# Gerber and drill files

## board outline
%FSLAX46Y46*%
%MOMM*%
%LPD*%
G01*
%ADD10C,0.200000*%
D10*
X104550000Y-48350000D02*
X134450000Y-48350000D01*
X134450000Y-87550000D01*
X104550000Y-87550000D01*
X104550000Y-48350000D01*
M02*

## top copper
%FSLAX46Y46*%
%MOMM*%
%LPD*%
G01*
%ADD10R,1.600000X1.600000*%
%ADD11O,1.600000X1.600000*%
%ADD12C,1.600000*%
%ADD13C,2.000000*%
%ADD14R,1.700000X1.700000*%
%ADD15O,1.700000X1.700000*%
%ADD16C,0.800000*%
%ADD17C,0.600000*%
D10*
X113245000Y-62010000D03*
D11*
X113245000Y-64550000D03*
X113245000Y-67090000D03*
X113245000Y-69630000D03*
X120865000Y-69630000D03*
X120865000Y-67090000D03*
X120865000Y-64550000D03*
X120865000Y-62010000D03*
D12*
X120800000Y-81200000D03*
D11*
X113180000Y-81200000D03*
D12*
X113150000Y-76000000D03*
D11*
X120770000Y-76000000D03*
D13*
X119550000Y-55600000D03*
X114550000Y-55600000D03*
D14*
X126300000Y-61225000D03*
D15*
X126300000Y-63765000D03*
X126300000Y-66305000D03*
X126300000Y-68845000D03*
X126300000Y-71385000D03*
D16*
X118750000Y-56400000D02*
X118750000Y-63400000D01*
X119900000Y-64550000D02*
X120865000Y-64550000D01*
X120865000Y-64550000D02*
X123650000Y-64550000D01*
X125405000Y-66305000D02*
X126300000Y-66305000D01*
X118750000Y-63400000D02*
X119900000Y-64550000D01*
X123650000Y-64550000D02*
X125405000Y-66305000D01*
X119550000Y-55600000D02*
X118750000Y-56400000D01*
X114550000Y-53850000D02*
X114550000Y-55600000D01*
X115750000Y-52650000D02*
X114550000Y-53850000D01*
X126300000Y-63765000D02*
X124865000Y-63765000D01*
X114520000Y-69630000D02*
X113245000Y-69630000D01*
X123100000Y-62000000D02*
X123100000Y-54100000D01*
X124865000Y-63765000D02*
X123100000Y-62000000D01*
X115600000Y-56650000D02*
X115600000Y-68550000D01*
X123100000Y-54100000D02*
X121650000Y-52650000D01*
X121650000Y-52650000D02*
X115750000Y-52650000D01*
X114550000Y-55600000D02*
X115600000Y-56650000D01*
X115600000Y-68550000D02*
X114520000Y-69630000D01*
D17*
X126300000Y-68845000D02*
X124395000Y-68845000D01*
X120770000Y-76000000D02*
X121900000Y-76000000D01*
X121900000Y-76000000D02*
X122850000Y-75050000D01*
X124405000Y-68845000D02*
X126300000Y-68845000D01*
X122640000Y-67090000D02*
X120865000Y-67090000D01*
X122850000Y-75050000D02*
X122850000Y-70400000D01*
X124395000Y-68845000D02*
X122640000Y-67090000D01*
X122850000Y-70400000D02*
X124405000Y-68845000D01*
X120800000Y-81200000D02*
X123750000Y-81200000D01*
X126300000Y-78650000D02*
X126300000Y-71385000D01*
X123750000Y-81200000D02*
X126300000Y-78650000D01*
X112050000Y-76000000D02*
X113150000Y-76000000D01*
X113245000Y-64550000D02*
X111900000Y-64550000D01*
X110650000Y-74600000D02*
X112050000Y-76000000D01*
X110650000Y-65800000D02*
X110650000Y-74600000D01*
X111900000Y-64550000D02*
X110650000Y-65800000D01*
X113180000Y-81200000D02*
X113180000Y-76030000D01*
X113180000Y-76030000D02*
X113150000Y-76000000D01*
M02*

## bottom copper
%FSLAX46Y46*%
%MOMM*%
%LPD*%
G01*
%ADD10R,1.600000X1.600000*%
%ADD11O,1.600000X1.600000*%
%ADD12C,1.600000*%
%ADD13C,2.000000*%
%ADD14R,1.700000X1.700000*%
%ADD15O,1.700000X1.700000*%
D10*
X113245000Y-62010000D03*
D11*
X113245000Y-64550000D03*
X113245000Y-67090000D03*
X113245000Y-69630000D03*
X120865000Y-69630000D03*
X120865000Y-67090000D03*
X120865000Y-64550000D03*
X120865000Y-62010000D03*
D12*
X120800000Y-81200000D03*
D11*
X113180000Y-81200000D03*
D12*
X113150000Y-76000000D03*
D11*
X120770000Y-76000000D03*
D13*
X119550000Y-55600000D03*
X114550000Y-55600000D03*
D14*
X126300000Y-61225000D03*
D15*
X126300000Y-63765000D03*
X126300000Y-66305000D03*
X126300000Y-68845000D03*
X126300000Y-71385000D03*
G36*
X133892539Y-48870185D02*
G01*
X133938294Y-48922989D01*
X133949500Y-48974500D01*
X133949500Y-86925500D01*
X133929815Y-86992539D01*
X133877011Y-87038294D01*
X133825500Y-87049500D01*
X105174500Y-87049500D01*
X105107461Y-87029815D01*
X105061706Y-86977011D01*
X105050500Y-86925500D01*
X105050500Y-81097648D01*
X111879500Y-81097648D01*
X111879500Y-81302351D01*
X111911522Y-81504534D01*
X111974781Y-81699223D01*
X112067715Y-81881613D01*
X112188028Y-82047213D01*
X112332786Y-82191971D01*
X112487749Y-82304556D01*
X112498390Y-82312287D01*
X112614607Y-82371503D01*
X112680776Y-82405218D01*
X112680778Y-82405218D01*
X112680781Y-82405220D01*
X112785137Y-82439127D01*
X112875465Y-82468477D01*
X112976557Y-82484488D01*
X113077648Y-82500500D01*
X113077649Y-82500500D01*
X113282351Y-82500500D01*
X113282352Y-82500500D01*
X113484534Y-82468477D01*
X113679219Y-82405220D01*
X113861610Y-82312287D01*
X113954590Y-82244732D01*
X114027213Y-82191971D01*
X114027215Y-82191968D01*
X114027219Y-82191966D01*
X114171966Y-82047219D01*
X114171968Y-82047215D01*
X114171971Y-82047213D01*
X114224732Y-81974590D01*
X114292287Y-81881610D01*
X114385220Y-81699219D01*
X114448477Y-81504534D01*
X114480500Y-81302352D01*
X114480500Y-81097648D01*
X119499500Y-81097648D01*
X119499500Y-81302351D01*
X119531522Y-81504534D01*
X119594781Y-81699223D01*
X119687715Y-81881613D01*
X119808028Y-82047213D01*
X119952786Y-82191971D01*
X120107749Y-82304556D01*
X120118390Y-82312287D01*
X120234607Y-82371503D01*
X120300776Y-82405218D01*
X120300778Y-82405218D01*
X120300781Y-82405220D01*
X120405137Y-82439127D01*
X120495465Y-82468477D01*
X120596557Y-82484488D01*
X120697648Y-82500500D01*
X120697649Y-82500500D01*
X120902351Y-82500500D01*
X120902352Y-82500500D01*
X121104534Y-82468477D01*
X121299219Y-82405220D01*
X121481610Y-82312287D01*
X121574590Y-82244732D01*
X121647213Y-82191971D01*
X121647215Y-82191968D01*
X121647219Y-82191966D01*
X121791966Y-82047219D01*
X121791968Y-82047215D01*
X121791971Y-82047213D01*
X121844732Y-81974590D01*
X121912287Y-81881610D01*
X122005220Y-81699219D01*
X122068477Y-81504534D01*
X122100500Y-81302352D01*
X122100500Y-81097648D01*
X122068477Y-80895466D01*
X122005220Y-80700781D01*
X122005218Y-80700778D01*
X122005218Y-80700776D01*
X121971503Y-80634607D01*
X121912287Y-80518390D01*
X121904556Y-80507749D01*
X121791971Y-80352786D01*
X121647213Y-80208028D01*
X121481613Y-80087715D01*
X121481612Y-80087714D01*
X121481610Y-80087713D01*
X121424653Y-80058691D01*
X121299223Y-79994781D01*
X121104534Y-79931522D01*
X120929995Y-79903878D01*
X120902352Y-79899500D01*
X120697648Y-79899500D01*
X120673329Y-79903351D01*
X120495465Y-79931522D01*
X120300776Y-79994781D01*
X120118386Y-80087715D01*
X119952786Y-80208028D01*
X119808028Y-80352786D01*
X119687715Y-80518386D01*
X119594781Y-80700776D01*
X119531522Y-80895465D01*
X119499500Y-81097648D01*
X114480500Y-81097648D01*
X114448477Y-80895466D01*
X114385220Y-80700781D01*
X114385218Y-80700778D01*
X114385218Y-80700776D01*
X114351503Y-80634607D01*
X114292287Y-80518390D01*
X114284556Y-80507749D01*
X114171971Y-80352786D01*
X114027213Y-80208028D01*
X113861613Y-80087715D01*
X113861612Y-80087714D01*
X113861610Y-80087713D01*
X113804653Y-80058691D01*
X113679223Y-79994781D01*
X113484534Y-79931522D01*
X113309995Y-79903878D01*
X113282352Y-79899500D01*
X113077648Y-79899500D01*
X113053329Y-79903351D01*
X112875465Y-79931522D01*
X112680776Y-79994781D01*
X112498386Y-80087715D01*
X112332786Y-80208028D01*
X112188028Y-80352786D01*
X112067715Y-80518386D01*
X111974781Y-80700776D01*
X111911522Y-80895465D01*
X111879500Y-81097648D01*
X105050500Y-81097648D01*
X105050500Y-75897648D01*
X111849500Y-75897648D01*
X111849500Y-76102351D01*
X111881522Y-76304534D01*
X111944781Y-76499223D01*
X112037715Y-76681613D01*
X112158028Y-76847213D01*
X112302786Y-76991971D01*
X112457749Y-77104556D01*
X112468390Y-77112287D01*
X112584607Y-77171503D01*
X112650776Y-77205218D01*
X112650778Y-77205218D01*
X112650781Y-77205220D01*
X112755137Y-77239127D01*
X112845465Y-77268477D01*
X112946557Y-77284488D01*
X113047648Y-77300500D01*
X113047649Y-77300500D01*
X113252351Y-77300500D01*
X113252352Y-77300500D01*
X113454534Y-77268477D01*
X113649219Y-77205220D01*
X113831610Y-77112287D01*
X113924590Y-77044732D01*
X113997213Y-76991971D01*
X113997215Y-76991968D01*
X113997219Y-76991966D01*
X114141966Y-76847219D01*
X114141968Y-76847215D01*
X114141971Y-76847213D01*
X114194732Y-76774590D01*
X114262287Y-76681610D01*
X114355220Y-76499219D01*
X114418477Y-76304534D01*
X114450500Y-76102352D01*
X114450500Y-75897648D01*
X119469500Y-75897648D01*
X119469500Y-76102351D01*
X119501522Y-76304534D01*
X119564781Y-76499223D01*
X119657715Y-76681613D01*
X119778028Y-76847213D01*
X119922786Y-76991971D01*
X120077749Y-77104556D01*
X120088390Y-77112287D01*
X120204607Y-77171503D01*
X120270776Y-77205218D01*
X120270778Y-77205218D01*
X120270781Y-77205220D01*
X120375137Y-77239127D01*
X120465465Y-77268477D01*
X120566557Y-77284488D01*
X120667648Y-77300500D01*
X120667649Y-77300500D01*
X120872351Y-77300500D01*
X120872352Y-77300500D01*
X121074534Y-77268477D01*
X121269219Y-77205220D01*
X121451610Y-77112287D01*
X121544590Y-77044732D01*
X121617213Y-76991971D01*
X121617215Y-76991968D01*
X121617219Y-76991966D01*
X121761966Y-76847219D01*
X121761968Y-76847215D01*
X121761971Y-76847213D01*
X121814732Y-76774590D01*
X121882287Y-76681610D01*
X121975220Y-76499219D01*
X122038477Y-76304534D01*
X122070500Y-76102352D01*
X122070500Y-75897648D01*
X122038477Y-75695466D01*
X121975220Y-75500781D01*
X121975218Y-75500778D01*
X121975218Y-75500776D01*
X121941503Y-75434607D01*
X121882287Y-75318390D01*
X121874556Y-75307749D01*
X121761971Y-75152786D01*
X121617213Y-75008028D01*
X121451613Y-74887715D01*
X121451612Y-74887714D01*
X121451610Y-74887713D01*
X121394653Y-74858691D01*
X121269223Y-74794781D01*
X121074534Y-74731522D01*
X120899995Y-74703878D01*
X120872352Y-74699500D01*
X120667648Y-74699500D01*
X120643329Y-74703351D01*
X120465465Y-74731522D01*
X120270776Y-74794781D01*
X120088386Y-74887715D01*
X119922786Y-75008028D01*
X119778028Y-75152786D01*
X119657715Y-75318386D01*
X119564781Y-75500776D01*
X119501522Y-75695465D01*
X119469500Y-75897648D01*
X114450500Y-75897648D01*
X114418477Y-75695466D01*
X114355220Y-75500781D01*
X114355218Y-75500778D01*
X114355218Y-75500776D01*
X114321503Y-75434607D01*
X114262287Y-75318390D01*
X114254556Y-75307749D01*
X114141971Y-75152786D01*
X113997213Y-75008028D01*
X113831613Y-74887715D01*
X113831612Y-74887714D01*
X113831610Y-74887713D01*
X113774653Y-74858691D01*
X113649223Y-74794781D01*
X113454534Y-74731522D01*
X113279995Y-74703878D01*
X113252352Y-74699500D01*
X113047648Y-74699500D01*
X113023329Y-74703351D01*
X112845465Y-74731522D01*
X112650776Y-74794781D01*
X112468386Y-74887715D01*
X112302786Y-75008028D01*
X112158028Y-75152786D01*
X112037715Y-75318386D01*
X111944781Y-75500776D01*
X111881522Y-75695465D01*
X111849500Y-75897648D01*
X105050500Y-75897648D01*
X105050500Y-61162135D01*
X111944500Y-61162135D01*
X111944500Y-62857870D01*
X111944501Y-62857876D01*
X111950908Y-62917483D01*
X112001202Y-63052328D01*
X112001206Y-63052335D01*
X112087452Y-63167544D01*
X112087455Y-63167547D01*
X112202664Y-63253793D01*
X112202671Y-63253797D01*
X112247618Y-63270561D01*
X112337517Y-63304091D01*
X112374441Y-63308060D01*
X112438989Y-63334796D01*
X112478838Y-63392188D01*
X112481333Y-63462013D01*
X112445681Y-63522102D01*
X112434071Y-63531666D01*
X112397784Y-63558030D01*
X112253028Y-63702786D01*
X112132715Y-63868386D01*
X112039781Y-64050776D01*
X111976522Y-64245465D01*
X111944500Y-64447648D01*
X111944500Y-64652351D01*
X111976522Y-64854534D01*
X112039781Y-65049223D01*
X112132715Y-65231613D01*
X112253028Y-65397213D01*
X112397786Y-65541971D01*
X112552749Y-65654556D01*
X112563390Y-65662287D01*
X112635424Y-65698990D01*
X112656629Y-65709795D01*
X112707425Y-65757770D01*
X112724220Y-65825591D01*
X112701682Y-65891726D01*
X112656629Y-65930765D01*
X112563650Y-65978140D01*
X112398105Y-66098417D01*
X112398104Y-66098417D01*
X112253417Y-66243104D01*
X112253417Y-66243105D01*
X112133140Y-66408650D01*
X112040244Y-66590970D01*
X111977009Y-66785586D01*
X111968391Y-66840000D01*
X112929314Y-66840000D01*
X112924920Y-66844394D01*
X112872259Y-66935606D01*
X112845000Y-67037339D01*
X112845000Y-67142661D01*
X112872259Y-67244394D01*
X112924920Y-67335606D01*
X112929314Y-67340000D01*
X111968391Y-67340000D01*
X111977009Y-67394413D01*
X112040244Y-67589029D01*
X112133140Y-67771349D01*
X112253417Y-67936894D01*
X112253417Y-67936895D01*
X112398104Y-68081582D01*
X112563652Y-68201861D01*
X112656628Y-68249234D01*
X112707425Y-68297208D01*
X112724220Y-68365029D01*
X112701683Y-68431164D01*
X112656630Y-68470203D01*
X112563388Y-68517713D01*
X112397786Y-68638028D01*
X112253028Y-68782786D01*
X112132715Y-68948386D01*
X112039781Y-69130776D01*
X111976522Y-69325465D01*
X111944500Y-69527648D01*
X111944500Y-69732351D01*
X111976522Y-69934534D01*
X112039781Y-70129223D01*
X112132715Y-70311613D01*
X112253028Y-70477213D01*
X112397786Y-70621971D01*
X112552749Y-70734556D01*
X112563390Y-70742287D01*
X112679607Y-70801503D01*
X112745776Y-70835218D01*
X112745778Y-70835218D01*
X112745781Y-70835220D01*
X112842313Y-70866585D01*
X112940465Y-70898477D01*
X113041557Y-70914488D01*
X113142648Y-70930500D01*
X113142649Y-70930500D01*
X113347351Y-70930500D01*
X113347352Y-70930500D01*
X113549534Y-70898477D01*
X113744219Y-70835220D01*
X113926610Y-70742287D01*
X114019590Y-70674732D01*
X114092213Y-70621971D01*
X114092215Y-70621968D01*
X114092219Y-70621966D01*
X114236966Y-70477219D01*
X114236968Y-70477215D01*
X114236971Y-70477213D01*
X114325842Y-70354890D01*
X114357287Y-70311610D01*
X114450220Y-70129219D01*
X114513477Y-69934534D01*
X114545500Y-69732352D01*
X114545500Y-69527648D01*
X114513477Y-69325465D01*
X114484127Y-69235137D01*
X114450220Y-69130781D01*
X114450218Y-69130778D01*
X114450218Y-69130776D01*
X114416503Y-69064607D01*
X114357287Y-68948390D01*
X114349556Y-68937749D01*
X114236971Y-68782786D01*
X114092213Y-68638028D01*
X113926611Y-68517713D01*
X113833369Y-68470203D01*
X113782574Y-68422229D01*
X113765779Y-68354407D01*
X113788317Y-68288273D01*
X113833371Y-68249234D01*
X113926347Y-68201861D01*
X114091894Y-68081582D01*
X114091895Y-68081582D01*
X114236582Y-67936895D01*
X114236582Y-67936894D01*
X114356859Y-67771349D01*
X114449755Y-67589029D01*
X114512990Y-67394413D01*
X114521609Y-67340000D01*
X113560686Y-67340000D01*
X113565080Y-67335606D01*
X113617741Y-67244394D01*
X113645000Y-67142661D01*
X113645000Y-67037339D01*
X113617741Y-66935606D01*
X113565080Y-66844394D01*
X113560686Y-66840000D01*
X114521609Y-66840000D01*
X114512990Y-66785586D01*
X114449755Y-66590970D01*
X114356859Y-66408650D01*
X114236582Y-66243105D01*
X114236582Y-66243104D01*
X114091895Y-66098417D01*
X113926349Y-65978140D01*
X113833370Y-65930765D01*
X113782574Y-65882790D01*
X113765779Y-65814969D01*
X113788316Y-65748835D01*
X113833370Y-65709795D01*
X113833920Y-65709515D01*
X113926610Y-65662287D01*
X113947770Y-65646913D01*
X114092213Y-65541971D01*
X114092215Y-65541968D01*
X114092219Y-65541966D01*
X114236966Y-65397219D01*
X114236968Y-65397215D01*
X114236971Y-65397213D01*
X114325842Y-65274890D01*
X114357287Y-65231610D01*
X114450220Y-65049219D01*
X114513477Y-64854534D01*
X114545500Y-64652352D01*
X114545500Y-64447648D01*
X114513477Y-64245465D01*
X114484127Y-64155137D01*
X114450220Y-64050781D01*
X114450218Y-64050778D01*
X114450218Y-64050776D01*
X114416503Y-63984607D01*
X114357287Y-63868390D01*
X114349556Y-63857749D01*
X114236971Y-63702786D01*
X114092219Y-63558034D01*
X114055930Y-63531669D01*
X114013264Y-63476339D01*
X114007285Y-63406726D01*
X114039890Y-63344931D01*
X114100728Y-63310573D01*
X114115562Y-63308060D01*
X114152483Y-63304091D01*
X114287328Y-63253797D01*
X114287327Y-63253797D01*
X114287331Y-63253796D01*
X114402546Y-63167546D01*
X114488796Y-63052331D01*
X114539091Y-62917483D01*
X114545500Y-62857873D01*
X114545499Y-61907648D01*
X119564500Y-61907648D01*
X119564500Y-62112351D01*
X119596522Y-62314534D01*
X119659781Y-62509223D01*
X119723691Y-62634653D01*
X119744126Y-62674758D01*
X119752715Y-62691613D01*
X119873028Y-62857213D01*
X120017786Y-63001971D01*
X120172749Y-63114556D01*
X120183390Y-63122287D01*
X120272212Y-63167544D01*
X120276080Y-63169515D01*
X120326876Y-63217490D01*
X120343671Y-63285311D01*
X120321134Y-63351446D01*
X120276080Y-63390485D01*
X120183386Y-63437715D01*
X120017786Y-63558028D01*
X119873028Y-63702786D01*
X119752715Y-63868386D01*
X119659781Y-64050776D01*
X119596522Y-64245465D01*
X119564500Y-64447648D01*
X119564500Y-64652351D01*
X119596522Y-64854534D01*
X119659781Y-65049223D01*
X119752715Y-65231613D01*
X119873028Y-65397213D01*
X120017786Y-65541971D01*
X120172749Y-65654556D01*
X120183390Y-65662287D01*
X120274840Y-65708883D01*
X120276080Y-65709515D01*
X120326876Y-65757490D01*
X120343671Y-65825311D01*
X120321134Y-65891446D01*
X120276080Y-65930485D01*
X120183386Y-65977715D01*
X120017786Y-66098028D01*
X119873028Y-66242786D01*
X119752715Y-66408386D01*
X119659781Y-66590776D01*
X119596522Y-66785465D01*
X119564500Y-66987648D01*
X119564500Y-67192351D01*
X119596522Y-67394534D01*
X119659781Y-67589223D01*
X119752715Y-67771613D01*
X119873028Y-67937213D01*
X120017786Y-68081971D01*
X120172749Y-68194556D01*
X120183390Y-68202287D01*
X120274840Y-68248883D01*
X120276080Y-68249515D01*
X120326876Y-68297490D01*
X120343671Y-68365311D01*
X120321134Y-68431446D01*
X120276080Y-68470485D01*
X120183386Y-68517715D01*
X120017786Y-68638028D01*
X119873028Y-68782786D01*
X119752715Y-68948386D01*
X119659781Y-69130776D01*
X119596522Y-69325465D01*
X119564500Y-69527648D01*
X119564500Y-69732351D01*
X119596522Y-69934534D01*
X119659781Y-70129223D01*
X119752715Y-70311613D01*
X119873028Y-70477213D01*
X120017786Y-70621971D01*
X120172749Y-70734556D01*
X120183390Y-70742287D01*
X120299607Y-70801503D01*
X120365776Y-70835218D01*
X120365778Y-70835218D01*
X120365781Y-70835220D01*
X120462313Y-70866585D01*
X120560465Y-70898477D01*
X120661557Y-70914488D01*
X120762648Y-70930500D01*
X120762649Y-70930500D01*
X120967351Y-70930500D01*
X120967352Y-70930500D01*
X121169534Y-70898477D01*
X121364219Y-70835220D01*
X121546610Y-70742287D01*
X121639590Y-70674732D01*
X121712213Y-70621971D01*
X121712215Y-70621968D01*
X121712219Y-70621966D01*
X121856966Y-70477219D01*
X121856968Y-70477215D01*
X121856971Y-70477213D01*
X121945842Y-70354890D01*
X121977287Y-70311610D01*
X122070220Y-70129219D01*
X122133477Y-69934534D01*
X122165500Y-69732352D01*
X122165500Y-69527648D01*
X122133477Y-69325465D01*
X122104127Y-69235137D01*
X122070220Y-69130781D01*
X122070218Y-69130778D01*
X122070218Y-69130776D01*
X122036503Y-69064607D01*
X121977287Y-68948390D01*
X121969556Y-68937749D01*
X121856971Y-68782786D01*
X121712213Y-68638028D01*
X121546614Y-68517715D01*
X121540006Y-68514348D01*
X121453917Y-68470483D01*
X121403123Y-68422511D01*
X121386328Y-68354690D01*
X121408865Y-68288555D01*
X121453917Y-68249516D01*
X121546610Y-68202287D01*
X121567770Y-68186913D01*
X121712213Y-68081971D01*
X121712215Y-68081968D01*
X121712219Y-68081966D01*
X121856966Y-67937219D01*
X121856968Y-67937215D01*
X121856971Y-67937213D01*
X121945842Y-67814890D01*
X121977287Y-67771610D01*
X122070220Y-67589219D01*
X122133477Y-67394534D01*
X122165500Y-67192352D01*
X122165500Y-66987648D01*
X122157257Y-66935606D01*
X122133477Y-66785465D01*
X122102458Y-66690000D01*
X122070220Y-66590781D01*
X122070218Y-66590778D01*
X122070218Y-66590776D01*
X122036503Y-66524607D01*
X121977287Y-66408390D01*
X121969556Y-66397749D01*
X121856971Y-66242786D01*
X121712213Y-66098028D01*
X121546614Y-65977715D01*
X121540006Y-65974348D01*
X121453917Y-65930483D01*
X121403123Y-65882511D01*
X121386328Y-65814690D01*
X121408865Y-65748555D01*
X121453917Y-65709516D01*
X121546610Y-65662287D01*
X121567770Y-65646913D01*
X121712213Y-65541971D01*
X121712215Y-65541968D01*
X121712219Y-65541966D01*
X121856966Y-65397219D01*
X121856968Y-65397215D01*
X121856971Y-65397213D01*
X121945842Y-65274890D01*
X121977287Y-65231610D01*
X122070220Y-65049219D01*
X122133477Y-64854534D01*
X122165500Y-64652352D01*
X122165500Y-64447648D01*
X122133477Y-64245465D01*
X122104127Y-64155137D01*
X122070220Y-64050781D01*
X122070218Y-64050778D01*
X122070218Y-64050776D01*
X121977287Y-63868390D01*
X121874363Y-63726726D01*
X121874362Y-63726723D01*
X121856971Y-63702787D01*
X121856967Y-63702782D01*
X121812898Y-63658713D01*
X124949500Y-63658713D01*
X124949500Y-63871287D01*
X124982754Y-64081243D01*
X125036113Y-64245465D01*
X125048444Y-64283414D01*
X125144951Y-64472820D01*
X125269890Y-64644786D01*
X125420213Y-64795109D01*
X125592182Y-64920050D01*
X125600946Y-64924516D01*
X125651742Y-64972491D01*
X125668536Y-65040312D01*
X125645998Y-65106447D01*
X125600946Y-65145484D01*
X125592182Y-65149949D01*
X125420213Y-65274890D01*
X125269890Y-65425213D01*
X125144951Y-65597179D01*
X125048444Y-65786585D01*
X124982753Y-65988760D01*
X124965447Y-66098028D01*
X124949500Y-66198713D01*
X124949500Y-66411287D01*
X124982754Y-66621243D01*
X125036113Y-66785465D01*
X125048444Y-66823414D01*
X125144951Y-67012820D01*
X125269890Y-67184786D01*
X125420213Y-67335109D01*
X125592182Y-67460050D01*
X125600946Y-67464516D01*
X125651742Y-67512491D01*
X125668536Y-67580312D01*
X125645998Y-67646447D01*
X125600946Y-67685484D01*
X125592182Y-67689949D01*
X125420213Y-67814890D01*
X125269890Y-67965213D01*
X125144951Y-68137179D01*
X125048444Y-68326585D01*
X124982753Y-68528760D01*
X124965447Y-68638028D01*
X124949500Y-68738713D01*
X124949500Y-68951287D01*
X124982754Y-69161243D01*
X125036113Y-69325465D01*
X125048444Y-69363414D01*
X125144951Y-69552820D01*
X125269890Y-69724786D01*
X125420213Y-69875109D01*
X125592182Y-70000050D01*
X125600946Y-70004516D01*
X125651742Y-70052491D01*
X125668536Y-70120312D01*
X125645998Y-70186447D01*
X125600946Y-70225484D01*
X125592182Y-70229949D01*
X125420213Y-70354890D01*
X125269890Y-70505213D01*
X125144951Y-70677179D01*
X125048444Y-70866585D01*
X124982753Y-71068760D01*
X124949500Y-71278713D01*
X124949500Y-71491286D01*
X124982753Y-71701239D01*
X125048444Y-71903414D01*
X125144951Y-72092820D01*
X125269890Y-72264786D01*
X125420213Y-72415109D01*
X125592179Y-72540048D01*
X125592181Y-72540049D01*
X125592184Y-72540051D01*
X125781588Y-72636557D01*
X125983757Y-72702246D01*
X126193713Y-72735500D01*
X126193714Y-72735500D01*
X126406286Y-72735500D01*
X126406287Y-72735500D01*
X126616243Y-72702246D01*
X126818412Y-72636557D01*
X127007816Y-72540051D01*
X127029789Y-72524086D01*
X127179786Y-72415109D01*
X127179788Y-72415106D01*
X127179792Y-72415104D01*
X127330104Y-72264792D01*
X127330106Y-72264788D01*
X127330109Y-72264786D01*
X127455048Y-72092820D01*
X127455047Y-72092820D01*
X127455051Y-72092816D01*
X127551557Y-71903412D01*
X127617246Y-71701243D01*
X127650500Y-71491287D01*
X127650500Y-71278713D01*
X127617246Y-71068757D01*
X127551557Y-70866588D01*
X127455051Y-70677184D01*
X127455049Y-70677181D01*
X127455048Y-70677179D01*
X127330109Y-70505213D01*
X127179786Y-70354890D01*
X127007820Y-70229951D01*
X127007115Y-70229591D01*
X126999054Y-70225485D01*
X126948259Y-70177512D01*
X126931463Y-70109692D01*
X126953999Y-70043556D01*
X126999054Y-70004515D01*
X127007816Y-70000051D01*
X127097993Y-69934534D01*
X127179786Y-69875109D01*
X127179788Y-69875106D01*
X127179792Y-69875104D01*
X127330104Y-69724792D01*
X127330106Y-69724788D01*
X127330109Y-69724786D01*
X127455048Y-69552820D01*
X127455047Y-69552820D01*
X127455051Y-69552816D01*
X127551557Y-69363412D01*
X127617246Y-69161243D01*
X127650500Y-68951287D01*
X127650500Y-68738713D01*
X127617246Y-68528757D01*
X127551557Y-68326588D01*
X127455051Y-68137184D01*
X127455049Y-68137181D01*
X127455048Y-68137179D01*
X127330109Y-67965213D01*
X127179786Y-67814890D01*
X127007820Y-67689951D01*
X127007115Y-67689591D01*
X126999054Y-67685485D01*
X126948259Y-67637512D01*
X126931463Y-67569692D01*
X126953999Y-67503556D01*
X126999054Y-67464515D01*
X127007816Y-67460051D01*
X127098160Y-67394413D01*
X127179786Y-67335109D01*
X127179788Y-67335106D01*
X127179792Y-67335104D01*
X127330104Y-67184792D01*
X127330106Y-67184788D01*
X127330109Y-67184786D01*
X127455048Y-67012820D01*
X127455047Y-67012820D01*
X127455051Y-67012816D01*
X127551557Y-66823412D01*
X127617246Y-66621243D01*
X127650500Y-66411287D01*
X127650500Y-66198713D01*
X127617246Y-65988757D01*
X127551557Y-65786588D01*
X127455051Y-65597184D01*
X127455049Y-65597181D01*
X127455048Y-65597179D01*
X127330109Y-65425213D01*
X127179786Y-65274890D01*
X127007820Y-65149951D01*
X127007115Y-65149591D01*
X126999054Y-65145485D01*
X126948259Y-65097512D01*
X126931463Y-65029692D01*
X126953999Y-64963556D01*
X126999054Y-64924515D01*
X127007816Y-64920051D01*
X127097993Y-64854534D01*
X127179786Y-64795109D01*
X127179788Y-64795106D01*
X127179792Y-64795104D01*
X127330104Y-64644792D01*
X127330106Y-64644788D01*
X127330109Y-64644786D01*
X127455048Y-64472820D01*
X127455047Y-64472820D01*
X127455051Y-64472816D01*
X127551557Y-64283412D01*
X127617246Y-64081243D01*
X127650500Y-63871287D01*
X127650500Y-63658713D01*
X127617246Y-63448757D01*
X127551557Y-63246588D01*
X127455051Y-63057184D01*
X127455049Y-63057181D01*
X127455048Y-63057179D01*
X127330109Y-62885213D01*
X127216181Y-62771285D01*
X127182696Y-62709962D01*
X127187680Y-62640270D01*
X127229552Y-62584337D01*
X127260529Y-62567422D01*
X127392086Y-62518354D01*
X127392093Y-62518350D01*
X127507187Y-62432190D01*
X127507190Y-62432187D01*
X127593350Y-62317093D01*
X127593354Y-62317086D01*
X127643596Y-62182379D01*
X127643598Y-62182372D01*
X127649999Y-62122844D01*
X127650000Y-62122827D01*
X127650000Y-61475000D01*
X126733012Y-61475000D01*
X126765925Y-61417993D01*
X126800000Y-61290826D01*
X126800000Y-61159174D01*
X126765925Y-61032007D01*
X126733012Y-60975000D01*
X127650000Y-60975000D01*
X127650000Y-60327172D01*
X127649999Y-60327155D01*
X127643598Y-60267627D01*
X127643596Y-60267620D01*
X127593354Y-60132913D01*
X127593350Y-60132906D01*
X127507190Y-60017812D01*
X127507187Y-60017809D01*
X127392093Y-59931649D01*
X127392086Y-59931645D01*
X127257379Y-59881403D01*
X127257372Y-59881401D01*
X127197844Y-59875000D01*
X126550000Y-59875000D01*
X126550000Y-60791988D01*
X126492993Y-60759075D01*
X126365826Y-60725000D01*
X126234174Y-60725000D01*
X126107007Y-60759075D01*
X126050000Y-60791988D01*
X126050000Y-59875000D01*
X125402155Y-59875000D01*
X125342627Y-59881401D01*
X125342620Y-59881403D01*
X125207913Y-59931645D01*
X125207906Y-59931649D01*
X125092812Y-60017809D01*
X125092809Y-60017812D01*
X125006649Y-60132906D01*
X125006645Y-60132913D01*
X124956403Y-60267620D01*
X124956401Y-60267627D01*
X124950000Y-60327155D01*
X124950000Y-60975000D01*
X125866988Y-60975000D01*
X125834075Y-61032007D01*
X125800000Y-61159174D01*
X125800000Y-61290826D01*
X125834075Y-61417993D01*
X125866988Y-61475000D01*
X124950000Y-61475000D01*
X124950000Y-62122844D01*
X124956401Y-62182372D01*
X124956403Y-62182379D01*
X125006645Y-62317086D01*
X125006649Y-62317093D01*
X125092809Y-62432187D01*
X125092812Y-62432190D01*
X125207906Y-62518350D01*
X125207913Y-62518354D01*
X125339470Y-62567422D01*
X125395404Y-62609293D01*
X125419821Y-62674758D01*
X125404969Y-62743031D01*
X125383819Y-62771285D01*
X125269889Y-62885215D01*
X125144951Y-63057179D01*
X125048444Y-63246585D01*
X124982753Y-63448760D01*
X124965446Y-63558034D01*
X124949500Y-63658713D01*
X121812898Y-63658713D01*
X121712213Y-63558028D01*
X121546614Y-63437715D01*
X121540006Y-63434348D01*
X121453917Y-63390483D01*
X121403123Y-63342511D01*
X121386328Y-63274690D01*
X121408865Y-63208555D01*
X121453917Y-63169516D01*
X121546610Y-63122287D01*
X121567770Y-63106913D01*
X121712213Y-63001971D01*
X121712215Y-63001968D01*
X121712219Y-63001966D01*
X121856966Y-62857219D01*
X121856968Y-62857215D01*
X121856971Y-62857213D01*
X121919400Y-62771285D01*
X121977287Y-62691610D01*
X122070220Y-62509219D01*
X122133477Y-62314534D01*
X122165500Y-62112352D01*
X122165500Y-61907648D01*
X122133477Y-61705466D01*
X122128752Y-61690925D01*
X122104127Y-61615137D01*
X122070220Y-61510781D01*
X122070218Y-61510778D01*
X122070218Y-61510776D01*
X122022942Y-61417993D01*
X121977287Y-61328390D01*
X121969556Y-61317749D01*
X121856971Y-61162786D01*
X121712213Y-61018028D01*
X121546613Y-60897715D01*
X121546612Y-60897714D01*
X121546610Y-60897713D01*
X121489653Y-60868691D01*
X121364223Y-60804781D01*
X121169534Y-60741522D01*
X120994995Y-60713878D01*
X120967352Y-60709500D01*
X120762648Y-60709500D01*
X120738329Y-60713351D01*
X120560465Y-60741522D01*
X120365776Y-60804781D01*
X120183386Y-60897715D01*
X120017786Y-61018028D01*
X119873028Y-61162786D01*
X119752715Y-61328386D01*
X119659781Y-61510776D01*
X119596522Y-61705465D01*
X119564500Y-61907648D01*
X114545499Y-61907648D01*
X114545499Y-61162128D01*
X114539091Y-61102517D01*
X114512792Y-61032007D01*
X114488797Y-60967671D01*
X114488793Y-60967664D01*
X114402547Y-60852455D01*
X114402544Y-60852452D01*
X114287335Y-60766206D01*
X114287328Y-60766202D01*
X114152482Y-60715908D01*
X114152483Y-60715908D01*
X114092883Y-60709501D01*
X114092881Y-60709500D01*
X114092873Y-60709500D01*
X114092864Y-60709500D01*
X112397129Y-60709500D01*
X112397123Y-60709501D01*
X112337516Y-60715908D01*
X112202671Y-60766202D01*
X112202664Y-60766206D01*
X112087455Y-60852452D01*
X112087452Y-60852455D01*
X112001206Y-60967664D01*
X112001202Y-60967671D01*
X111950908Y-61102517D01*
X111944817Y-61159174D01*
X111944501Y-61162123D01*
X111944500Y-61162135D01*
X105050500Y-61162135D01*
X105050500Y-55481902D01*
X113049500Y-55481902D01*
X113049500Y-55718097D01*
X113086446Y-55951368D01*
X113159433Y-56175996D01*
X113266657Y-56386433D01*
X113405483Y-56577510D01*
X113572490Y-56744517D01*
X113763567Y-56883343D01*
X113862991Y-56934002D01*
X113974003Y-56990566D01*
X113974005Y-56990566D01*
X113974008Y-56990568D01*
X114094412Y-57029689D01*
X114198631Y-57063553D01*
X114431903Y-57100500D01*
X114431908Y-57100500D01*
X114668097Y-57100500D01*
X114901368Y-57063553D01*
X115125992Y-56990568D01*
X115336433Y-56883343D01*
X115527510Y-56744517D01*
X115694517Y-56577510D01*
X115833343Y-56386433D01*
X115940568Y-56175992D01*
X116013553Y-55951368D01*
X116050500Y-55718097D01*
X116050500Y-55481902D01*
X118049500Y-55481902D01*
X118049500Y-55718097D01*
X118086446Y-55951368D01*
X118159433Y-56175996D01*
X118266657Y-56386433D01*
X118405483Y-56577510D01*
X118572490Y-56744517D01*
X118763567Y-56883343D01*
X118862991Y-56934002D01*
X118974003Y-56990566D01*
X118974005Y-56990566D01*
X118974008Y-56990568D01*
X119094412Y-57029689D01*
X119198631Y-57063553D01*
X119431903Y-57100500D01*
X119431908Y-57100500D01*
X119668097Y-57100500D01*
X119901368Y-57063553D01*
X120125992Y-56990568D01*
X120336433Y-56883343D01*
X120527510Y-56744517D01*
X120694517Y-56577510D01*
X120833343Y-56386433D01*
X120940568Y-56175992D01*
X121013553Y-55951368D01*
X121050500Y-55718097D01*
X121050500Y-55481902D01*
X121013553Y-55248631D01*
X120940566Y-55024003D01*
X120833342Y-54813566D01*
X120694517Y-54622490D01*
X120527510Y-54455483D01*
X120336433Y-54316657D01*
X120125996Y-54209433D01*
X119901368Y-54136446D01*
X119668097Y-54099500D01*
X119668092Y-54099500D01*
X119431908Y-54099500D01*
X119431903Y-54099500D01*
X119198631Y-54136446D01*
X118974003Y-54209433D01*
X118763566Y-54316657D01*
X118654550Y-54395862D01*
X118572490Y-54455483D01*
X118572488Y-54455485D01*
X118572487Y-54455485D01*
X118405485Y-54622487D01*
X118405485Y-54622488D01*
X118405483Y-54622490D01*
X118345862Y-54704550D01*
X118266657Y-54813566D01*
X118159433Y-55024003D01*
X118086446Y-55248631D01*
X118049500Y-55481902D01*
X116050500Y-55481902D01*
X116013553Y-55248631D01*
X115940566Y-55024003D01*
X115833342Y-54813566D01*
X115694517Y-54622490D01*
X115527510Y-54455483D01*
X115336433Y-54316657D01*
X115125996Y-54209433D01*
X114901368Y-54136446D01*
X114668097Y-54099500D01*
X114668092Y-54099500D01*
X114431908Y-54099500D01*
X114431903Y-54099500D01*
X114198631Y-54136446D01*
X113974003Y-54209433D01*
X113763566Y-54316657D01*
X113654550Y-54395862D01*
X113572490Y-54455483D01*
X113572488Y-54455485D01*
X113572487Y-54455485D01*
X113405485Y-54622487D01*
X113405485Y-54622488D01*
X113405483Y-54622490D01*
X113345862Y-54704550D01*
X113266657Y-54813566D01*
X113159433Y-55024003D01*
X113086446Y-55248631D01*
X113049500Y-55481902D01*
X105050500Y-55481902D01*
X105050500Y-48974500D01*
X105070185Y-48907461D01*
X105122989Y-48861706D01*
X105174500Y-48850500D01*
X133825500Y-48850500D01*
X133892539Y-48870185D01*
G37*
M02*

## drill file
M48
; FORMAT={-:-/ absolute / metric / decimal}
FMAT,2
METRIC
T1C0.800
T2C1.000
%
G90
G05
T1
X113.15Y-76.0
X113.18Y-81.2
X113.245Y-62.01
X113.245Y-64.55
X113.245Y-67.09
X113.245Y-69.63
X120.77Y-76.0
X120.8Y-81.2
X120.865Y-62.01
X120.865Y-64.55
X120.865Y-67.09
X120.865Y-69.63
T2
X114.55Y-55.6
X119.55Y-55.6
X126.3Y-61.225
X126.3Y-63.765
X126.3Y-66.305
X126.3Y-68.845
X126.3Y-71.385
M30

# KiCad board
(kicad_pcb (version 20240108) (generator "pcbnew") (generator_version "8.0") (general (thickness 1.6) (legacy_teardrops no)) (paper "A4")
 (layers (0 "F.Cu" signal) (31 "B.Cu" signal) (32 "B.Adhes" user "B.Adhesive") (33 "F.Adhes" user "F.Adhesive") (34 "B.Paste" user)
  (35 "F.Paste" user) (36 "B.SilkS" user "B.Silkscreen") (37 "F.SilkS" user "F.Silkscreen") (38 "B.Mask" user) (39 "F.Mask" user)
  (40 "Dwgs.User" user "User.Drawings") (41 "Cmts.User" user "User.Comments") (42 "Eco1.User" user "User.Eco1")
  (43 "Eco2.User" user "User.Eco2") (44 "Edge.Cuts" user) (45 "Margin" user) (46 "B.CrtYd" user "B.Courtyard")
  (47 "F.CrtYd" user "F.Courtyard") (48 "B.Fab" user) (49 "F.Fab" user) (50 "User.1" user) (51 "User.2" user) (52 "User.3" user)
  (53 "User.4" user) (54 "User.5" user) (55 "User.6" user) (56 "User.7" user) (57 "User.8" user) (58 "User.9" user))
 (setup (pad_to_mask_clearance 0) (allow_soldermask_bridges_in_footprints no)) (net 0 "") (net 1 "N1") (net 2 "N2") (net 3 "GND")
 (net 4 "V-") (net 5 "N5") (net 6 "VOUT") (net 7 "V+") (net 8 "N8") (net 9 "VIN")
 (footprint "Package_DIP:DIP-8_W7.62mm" (layer "F.Cu") (at 113.245 62.01)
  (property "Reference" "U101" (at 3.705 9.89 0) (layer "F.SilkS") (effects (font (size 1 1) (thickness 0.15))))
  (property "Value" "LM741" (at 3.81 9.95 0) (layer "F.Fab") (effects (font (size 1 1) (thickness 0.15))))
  (pad "1" thru_hole rect (at 0 0) (size 1.6 1.6) (drill 0.8) (layers "*.Cu" "*.Mask") (remove_unused_layers no) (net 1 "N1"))
  (pad "2" thru_hole oval (at 0 2.54) (size 1.6 1.6) (drill 0.8) (layers "*.Cu" "*.Mask") (remove_unused_layers no) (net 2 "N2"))
  (pad "3" thru_hole oval (at 0 5.08) (size 1.6 1.6) (drill 0.8) (layers "*.Cu" "*.Mask") (remove_unused_layers no) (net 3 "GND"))
  (pad "4" thru_hole oval (at 0 7.62) (size 1.6 1.6) (drill 0.8) (layers "*.Cu" "*.Mask") (remove_unused_layers no) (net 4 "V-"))
  (pad "5" thru_hole oval (at 7.62 7.62) (size 1.6 1.6) (drill 0.8) (layers "*.Cu" "*.Mask") (remove_unused_layers no) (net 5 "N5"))
  (pad "6" thru_hole oval (at 7.62 5.08) (size 1.6 1.6) (drill 0.8) (layers "*.Cu" "*.Mask") (remove_unused_layers no) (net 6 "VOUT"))
  (pad "7" thru_hole oval (at 7.62 2.54) (size 1.6 1.6) (drill 0.8) (layers "*.Cu" "*.Mask") (remove_unused_layers no) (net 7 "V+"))
  (pad "8" thru_hole oval (at 7.62 0) (size 1.6 1.6) (drill 0.8) (layers "*.Cu" "*.Mask") (remove_unused_layers no) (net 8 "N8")))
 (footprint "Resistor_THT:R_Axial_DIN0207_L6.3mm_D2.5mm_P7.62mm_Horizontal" (layer "F.Cu") (at 120.8 81.2 180)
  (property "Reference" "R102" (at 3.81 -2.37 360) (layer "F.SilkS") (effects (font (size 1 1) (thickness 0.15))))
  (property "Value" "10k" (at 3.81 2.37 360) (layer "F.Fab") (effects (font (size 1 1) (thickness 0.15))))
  (pad "1" thru_hole circle (at 0 0 180) (size 1.6 1.6) (drill 0.8) (layers "*.Cu" "*.Mask") (remove_unused_layers no) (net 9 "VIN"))
  (pad "2" thru_hole oval (at 7.62 0 180) (size 1.6 1.6) (drill 0.8) (layers "*.Cu" "*.Mask") (remove_unused_layers no) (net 2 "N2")))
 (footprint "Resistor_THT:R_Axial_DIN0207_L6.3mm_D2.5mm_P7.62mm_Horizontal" (layer "F.Cu") (at 113.15 76)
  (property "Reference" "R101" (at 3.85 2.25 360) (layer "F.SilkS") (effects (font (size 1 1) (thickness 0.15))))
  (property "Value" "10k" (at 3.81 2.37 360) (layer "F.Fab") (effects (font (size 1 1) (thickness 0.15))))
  (pad "1" thru_hole circle (at 0 0) (size 1.6 1.6) (drill 0.8) (layers "*.Cu" "*.Mask") (remove_unused_layers no) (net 2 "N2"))
  (pad "2" thru_hole oval (at 7.62 0) (size 1.6 1.6) (drill 0.8) (layers "*.Cu" "*.Mask") (remove_unused_layers no) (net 6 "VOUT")))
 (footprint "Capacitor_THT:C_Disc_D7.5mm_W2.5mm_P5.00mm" (layer "F.Cu") (at 119.55 55.6 180)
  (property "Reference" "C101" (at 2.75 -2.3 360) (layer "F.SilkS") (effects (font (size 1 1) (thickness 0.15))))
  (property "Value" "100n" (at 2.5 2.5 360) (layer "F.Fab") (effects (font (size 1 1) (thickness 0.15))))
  (pad "1" thru_hole circle (at 0 0 180) (size 2 2) (drill 1) (layers "*.Cu" "*.Mask") (remove_unused_layers no) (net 7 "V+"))
  (pad "2" thru_hole circle (at 5 0 180) (size 2 2) (drill 1) (layers "*.Cu" "*.Mask") (remove_unused_layers no) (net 4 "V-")))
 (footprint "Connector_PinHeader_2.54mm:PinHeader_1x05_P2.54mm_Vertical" (layer "F.Cu") (at 126.3 61.225)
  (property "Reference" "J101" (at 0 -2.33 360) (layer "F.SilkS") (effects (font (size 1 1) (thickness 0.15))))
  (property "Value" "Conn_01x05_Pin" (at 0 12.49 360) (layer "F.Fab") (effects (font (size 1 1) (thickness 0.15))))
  (pad "1" thru_hole rect (at 0 0) (size 1.7 1.7) (drill 1) (layers "*.Cu" "*.Mask") (remove_unused_layers no) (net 3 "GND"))
  (pad "2" thru_hole oval (at 0 2.54) (size 1.7 1.7) (drill 1) (layers "*.Cu" "*.Mask") (remove_unused_layers no) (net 4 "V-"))
  (pad "3" thru_hole oval (at 0 5.08) (size 1.7 1.7) (drill 1) (layers "*.Cu" "*.Mask") (remove_unused_layers no) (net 7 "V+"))
  (pad "4" thru_hole oval (at 0 7.62) (size 1.7 1.7) (drill 1) (layers "*.Cu" "*.Mask") (remove_unused_layers no) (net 6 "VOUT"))
  (pad "5" thru_hole oval (at 0 10.16) (size 1.7 1.7) (drill 1) (layers "*.Cu" "*.Mask") (remove_unused_layers no) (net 9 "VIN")))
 (gr_rect (start 104.55 48.35) (end 134.45 87.55) (stroke (width 0.2) (type default)) (fill none) (layer "Edge.Cuts"))
 (segment (start 118.75 56.4) (end 118.75 63.4) (width 0.8) (layer "F.Cu") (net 7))
 (segment (start 119.9 64.55) (end 120.865 64.55) (width 0.8) (layer "F.Cu") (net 7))
 (segment (start 120.865 64.55) (end 123.65 64.55) (width 0.8) (layer "F.Cu") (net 7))
 (segment (start 125.405 66.305) (end 126.3 66.305) (width 0.8) (layer "F.Cu") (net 7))
 (segment (start 118.75 63.4) (end 119.9 64.55) (width 0.8) (layer "F.Cu") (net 7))
 (segment (start 123.65 64.55) (end 125.405 66.305) (width 0.8) (layer "F.Cu") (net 7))
 (segment (start 119.55 55.6) (end 118.75 56.4) (width 0.8) (layer "F.Cu") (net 7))
 (segment (start 114.55 53.85) (end 114.55 55.6) (width 0.8) (layer "F.Cu") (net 4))
 (segment (start 115.75 52.65) (end 114.55 53.85) (width 0.8) (layer "F.Cu") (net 4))
 (segment (start 126.3 63.765) (end 124.865 63.765) (width 0.8) (layer "F.Cu") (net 4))
 (segment (start 114.52 69.63) (end 113.245 69.63) (width 0.8) (layer "F.Cu") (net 4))
 (segment (start 123.1 62) (end 123.1 54.1) (width 0.8) (layer "F.Cu") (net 4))
 (segment (start 124.865 63.765) (end 123.1 62) (width 0.8) (layer "F.Cu") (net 4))
 (segment (start 115.6 56.65) (end 115.6 68.55) (width 0.8) (layer "F.Cu") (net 4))
 (segment (start 123.1 54.1) (end 121.65 52.65) (width 0.8) (layer "F.Cu") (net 4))
 (segment (start 121.65 52.65) (end 115.75 52.65) (width 0.8) (layer "F.Cu") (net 4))
 (segment (start 114.55 55.6) (end 115.6 56.65) (width 0.8) (layer "F.Cu") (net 4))
 (segment (start 115.6 68.55) (end 114.52 69.63) (width 0.8) (layer "F.Cu") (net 4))
 (segment (start 126.3 68.845) (end 124.395 68.845) (width 0.6) (layer "F.Cu") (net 6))
 (segment (start 120.77 76) (end 121.9 76) (width 0.6) (layer "F.Cu") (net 6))
 (segment (start 121.9 76) (end 122.85 75.05) (width 0.6) (layer "F.Cu") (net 6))
 (segment (start 124.405 68.845) (end 126.3 68.845) (width 0.6) (layer "F.Cu") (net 6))
 (segment (start 122.64 67.09) (end 120.865 67.09) (width 0.6) (layer "F.Cu") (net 6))
 (segment (start 122.85 75.05) (end 122.85 70.4) (width 0.6) (layer "F.Cu") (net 6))
 (segment (start 124.395 68.845) (end 122.64 67.09) (width 0.6) (layer "F.Cu") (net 6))
 (segment (start 122.85 70.4) (end 124.405 68.845) (width 0.6) (layer "F.Cu") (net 6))
 (segment (start 120.8 81.2) (end 123.75 81.2) (width 0.6) (layer "F.Cu") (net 9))
 (segment (start 126.3 78.65) (end 126.3 71.385) (width 0.6) (layer "F.Cu") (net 9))
 (segment (start 123.75 81.2) (end 126.3 78.65) (width 0.6) (layer "F.Cu") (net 9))
 (segment (start 112.05 76) (end 113.15 76) (width 0.6) (layer "F.Cu") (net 2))
 (segment (start 113.245 64.55) (end 111.9 64.55) (width 0.6) (layer "F.Cu") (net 2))
 (segment (start 110.65 74.6) (end 112.05 76) (width 0.6) (layer "F.Cu") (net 2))
 (segment (start 110.65 65.8) (end 110.65 74.6) (width 0.6) (layer "F.Cu") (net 2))
 (segment (start 111.9 64.55) (end 110.65 65.8) (width 0.6) (layer "F.Cu") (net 2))
 (segment (start 113.18 81.2) (end 113.18 76.03) (width 0.6) (layer "F.Cu") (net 2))
 (segment (start 113.18 76.03) (end 113.15 76) (width 0.6) (layer "F.Cu") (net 2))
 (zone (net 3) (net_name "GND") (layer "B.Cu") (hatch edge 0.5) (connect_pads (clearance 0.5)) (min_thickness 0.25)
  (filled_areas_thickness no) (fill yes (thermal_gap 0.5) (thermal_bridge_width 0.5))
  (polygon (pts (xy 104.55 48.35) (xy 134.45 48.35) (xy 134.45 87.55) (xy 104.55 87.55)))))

